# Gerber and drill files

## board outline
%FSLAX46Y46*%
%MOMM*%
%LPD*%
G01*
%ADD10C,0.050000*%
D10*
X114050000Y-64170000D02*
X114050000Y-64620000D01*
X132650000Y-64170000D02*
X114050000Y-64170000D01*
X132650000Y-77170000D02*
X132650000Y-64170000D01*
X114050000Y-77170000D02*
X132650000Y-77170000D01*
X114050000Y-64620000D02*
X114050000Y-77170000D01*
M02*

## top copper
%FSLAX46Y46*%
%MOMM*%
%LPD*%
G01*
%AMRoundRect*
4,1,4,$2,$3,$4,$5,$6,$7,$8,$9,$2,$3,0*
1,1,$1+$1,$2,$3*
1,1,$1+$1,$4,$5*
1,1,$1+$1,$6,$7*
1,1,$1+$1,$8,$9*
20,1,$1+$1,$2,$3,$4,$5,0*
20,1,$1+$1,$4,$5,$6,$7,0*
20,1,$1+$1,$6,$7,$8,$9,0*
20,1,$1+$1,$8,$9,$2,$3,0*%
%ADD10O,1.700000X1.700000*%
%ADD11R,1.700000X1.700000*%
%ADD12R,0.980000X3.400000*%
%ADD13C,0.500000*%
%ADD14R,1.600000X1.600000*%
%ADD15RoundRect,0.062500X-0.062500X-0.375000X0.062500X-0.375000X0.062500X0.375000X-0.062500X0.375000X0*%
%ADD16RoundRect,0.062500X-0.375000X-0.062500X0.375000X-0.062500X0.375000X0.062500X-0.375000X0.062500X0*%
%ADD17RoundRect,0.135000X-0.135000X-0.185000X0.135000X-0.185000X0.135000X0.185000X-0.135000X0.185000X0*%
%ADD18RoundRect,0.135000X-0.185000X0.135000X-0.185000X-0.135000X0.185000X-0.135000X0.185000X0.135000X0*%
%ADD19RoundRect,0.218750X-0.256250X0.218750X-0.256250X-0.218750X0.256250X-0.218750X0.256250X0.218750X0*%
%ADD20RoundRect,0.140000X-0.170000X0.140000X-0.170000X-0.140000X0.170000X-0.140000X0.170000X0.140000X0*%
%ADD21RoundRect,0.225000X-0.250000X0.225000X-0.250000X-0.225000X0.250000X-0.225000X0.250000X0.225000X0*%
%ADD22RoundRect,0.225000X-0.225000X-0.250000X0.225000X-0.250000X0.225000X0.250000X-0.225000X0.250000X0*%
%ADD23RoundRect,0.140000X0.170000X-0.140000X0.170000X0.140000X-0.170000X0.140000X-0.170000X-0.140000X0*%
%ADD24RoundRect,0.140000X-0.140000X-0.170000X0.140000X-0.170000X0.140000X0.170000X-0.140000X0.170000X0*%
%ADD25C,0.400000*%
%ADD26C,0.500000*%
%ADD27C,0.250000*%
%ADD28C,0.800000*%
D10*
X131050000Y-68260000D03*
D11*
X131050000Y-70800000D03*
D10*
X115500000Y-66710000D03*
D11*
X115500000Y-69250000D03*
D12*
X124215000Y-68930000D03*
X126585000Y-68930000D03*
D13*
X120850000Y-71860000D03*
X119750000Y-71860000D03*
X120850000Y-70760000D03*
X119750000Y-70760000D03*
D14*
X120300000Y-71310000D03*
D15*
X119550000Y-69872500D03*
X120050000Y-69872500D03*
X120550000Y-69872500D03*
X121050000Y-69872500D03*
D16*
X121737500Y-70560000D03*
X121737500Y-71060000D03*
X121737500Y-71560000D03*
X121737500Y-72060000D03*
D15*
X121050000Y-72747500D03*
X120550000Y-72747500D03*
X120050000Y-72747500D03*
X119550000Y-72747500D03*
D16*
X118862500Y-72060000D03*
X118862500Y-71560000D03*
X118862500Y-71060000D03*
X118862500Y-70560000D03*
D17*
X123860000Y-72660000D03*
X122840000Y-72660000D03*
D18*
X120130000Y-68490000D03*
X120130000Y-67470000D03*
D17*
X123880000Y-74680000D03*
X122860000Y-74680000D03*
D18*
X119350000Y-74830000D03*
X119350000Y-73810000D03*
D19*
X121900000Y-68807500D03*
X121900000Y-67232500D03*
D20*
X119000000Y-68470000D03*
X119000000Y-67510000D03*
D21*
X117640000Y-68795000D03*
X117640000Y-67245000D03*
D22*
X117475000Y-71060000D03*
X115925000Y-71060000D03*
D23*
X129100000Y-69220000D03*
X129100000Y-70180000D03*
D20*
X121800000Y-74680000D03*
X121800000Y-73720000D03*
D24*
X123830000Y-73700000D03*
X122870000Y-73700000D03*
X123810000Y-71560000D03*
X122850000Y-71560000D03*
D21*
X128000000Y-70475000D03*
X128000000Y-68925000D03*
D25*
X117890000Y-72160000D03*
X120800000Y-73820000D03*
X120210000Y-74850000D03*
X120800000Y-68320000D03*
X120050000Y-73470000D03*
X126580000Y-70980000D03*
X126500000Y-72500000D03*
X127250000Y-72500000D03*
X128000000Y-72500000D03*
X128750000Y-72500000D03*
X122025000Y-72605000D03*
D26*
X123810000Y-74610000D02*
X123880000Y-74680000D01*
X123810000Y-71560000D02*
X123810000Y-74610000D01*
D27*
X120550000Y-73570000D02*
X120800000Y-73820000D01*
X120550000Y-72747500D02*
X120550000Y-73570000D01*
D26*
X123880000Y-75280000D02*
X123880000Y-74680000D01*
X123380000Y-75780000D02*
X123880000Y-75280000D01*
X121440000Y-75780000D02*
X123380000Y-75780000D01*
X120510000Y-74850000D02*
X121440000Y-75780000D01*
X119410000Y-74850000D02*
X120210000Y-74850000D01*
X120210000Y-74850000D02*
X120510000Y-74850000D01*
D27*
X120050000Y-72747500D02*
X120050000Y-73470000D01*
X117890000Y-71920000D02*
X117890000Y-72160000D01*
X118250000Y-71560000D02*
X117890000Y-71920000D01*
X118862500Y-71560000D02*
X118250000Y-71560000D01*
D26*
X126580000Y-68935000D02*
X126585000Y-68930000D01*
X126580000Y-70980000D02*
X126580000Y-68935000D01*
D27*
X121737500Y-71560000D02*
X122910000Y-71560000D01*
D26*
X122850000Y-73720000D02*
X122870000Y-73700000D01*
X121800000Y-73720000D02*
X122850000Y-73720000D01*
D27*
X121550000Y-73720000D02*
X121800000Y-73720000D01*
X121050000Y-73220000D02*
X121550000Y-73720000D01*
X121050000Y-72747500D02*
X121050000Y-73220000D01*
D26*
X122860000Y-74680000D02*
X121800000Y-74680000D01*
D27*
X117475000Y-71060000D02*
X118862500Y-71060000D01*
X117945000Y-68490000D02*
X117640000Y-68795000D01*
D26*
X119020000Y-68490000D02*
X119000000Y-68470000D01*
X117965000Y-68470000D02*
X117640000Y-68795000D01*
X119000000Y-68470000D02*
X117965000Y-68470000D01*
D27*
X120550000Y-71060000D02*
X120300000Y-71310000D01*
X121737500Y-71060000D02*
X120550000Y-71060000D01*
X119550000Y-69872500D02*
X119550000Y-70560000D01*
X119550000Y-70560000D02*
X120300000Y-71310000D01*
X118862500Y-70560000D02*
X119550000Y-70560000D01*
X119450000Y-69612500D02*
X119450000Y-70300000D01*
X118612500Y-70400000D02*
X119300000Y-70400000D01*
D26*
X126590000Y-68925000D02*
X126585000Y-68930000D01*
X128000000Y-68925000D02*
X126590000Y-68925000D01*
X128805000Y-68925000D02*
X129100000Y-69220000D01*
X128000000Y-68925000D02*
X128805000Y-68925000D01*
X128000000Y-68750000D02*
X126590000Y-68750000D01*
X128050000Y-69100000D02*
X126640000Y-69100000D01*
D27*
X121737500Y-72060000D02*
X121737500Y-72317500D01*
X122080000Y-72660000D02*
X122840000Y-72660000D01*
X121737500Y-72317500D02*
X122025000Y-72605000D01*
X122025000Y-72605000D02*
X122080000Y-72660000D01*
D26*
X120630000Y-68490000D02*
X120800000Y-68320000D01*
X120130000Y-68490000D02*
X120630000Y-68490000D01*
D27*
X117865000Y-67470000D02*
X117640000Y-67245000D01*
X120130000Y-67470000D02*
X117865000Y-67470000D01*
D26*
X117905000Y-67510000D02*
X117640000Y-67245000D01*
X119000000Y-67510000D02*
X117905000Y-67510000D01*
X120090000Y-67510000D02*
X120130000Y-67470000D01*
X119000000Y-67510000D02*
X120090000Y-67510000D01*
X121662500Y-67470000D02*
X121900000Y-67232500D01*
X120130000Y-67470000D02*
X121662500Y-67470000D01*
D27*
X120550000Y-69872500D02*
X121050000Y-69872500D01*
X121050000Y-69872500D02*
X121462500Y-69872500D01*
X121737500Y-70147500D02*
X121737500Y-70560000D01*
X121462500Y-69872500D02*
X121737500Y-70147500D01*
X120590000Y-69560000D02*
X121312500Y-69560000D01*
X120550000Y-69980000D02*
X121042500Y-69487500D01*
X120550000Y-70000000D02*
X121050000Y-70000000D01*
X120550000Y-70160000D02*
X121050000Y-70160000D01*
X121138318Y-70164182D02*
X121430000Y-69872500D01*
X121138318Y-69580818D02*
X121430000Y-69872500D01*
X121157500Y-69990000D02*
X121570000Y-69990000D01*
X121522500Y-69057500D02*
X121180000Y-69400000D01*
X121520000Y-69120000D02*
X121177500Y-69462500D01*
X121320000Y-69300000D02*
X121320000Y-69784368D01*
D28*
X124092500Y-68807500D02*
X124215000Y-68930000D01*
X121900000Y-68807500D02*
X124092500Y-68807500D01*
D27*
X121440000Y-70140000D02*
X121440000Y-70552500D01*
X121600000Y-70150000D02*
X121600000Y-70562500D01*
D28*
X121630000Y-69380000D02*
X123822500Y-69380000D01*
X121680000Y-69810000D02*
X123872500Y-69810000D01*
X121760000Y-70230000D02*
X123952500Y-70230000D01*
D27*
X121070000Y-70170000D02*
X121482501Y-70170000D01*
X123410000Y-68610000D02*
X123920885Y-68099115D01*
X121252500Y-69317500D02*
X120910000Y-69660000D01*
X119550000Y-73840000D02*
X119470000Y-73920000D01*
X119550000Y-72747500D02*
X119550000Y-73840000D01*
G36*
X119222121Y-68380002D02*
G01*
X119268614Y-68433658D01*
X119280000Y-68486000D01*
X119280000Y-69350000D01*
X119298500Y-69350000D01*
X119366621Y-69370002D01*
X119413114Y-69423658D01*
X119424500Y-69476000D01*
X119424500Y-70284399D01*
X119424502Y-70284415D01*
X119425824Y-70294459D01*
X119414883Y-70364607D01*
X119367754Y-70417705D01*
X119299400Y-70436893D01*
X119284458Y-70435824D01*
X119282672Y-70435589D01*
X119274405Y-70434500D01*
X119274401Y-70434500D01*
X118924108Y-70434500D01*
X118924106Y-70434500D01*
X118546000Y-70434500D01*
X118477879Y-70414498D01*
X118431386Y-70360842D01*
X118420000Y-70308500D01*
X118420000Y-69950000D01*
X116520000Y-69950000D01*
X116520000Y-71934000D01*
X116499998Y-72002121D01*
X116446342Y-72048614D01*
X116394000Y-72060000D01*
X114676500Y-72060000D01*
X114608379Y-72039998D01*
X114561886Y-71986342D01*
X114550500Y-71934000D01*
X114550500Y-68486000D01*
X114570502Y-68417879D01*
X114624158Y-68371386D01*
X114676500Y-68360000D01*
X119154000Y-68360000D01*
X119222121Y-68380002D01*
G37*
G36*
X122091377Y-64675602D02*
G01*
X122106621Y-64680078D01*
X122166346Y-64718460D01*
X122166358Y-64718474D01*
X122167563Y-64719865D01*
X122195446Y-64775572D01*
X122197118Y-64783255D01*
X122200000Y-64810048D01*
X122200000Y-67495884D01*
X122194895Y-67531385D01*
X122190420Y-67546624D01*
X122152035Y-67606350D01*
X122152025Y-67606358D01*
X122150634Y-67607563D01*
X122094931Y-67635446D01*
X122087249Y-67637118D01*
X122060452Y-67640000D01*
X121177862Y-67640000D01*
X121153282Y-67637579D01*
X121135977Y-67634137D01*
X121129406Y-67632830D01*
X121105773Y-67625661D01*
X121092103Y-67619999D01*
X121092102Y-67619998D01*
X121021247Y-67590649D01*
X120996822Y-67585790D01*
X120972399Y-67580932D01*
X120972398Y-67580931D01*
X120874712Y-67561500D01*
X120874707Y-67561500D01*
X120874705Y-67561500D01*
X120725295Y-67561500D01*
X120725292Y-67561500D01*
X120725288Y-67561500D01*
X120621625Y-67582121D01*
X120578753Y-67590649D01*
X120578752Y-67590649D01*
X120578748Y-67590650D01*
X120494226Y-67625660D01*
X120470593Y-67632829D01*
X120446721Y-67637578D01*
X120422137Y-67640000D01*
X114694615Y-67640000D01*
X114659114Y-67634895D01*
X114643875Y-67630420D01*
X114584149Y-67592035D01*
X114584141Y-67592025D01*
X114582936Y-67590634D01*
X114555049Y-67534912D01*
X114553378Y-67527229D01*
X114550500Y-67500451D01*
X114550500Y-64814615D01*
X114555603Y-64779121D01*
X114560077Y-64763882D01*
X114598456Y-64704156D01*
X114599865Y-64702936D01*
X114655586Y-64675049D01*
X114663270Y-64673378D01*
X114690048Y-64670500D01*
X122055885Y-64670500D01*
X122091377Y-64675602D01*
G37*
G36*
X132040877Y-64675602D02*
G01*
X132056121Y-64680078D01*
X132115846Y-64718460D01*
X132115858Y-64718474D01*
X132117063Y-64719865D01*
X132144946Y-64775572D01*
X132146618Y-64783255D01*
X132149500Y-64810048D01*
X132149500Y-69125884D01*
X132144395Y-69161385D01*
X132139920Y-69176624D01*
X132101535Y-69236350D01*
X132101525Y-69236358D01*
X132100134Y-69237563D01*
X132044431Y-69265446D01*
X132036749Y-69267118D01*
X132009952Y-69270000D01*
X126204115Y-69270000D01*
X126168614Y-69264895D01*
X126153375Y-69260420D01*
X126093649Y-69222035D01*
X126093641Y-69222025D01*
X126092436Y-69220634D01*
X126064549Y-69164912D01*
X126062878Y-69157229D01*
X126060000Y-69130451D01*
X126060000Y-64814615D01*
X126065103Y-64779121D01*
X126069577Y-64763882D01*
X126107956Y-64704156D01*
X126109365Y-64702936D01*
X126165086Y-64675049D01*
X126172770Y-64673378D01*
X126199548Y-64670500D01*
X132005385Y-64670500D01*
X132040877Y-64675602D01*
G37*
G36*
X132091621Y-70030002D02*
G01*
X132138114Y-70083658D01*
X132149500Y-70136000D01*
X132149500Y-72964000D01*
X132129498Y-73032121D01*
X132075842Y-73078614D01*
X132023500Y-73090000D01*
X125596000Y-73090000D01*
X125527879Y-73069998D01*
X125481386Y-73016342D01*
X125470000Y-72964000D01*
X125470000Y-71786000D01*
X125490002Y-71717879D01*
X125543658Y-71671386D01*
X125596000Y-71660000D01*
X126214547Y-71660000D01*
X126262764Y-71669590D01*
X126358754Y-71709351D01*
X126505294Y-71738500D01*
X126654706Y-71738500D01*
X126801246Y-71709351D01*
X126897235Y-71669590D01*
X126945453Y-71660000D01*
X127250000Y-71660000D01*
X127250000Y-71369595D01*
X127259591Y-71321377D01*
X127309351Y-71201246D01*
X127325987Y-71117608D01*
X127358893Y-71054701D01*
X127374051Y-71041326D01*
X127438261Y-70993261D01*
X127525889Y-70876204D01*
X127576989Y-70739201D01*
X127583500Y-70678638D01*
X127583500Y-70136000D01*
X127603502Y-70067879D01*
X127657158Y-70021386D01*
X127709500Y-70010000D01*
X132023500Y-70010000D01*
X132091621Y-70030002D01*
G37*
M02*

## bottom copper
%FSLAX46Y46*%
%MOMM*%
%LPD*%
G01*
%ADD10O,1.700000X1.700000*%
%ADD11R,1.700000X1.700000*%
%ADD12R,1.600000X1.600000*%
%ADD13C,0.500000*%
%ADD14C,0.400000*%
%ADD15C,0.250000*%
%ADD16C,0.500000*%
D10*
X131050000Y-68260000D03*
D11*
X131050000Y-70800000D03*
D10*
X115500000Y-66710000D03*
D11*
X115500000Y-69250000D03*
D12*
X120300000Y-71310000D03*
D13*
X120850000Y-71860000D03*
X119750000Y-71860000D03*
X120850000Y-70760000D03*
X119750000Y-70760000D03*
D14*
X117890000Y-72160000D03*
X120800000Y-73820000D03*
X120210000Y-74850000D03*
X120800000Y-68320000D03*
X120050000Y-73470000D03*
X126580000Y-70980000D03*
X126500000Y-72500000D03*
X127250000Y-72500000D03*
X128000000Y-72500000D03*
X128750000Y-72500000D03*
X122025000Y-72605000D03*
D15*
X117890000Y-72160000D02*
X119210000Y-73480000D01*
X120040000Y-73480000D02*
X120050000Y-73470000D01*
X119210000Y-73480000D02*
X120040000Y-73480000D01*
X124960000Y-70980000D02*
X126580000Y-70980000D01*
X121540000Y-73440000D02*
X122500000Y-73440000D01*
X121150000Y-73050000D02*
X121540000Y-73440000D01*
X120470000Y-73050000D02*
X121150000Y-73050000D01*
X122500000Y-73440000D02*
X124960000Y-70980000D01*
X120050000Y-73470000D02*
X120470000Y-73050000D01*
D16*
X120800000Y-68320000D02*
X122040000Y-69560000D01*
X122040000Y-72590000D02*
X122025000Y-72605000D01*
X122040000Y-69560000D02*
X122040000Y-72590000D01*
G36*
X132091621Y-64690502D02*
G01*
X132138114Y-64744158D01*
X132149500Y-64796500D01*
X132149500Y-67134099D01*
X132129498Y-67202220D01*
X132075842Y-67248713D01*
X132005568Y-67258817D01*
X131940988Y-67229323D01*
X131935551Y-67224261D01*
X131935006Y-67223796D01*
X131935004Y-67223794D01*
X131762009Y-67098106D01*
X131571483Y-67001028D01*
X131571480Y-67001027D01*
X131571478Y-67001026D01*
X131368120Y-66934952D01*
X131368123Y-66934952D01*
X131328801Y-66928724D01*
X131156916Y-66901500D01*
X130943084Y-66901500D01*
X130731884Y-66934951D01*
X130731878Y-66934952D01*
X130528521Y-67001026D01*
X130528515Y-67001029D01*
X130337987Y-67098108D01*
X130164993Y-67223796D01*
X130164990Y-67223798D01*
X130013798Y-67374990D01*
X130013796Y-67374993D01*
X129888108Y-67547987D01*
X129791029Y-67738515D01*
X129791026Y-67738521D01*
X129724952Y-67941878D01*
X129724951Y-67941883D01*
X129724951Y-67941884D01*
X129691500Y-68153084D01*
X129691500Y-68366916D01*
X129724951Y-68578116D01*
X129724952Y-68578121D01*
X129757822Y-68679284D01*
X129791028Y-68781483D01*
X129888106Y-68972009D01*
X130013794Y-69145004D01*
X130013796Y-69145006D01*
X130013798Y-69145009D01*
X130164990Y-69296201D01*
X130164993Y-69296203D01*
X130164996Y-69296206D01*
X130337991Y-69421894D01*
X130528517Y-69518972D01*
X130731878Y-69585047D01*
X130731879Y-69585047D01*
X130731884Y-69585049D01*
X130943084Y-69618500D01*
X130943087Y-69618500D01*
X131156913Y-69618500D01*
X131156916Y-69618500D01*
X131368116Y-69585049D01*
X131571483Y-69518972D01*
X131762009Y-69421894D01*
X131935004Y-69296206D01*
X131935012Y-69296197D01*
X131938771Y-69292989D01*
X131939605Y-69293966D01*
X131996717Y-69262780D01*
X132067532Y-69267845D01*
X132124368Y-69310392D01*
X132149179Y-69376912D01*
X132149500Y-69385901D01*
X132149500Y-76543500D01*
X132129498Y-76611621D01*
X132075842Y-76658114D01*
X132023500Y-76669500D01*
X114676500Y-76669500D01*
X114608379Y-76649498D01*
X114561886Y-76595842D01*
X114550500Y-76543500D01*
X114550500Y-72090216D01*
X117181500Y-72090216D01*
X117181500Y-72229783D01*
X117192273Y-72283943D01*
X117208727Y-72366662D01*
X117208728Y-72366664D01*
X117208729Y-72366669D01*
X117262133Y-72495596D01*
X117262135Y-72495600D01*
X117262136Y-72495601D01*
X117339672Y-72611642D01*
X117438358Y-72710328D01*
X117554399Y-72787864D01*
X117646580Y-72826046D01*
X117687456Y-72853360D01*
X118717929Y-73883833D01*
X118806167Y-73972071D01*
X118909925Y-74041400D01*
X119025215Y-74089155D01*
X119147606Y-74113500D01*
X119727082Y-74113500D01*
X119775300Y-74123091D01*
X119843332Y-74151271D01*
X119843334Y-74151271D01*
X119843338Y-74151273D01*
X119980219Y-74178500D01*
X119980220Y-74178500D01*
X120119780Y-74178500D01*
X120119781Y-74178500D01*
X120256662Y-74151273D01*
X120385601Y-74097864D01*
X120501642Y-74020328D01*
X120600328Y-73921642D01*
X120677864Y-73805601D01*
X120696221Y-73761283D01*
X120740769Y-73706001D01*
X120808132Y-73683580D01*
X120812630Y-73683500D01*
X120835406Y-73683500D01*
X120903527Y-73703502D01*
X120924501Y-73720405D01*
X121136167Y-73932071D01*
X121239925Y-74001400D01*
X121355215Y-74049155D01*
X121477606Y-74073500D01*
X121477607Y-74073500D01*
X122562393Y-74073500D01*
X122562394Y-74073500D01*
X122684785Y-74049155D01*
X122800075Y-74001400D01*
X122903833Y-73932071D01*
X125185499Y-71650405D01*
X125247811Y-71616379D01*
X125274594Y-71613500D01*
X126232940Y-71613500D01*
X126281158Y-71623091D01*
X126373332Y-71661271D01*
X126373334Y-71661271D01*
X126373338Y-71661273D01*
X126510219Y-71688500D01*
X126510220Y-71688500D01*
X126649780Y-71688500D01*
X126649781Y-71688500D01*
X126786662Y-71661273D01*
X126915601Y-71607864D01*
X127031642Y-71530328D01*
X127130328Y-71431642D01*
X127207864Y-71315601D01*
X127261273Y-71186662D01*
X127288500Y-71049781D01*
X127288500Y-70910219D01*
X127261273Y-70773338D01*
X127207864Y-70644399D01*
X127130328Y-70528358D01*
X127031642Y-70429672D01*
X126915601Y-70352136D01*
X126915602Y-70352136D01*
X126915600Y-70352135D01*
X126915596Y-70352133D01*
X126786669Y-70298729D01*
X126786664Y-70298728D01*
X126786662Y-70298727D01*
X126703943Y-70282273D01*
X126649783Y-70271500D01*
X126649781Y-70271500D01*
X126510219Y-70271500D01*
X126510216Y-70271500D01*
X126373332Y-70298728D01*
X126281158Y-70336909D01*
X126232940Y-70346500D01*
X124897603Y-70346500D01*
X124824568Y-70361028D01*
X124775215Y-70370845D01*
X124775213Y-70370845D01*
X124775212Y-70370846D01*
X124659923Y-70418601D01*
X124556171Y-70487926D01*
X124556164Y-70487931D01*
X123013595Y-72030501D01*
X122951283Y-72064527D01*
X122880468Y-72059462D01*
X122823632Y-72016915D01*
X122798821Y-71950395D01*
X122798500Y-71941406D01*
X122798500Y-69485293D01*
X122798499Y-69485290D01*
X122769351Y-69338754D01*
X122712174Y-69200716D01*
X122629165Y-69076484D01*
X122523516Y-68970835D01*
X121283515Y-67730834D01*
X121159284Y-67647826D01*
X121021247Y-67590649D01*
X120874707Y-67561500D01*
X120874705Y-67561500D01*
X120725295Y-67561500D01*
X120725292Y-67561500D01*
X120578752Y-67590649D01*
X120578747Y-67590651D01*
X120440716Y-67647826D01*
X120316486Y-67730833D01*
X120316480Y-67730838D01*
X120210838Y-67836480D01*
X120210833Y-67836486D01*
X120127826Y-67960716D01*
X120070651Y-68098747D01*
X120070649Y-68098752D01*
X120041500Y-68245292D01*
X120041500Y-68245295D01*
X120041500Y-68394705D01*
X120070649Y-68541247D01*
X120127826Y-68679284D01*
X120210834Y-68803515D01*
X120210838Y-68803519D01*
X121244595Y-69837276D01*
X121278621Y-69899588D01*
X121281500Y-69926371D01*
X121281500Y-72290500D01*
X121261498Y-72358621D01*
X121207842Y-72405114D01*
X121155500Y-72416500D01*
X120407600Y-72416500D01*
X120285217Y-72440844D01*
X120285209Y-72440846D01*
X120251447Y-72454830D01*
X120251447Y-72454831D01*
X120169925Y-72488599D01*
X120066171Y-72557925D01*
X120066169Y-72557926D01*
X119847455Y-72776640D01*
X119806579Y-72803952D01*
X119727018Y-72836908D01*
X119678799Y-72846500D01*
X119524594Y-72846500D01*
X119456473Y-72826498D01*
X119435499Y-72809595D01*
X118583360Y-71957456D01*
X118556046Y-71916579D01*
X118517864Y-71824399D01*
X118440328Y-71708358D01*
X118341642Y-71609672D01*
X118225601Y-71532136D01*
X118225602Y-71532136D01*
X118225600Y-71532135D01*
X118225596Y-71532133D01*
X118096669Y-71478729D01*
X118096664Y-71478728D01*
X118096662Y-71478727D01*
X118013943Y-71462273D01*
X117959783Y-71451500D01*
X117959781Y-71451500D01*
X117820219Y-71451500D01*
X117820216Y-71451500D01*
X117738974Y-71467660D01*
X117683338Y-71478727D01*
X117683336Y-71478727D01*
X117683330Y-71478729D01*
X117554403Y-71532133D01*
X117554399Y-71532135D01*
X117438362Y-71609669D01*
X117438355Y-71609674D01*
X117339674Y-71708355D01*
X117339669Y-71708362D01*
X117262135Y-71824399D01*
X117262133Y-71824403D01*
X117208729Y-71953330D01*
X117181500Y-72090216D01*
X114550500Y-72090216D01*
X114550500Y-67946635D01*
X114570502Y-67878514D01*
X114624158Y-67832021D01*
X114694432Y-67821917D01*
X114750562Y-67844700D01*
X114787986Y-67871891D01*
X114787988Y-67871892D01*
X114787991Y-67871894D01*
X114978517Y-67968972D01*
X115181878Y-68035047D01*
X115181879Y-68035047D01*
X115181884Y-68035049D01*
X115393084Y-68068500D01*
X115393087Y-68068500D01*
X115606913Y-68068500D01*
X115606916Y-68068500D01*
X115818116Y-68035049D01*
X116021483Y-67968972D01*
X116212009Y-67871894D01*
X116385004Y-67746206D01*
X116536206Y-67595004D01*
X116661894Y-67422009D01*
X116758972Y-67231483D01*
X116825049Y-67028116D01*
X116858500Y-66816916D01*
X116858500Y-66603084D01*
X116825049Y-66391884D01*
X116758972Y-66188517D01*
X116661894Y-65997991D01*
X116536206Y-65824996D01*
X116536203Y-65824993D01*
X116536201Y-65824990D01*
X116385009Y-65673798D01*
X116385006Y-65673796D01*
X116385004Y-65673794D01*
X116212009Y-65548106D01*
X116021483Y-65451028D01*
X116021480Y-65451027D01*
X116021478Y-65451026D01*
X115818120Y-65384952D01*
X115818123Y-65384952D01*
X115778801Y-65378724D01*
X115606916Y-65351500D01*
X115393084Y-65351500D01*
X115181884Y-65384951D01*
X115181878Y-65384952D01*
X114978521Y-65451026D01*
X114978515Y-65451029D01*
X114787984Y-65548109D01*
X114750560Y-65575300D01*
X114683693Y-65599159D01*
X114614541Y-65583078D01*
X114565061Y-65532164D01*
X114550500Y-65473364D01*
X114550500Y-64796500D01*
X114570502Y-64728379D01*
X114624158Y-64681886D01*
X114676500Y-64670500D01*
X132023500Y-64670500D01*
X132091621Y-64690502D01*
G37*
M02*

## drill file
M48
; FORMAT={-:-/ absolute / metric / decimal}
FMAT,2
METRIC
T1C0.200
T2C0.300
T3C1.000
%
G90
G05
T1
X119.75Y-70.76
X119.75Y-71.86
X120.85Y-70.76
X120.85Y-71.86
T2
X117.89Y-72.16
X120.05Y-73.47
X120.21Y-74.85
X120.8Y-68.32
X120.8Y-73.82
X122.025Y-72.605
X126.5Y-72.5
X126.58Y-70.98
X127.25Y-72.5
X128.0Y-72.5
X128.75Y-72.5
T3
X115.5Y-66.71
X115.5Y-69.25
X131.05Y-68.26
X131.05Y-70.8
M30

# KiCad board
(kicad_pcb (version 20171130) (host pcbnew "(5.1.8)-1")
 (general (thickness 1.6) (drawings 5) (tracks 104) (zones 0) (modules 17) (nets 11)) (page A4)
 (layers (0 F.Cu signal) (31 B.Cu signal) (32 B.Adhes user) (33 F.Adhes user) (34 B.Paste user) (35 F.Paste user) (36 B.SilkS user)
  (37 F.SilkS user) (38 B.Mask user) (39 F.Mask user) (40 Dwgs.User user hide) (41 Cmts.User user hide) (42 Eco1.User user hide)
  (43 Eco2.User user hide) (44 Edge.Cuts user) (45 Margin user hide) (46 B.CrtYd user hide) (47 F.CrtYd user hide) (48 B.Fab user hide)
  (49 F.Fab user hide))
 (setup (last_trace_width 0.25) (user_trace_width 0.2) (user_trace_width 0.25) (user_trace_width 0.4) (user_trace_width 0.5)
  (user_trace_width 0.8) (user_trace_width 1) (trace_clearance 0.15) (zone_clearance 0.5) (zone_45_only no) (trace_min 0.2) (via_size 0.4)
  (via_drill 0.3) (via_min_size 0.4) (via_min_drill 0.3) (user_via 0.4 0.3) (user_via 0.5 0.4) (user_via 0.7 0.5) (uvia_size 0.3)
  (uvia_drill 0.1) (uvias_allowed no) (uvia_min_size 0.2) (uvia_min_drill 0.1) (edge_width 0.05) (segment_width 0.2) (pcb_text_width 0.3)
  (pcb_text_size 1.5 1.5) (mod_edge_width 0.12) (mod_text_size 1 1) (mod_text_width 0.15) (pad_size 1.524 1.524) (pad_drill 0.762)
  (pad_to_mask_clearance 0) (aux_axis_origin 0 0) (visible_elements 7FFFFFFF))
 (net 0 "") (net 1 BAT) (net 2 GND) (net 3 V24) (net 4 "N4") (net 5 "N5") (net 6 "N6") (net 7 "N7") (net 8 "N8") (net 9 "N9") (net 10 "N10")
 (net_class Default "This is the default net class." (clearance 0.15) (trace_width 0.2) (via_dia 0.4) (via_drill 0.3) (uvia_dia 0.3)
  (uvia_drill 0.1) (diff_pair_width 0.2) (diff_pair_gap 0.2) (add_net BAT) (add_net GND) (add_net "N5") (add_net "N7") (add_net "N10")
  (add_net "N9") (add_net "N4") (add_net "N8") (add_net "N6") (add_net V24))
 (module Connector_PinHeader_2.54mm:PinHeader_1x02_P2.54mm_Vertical (layer F.Cu) (at 131.05 70.8 180)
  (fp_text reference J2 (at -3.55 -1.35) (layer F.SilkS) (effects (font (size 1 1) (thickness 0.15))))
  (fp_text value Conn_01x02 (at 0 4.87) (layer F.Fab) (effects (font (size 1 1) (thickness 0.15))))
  (pad 2 thru_hole oval (at 0 2.54 180) (size 1.7 1.7) (drill 1) (layers *.Cu *.Mask) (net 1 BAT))
  (pad 1 thru_hole rect (at 0 0 180) (size 1.7 1.7) (drill 1) (layers *.Cu *.Mask) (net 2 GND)))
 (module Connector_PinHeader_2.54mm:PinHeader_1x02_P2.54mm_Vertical (layer F.Cu) (at 115.5 69.25 180)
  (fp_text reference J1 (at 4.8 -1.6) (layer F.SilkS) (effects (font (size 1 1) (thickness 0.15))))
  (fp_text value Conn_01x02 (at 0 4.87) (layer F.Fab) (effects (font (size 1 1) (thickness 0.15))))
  (pad 2 thru_hole oval (at 0 2.54 180) (size 1.7 1.7) (drill 1) (layers *.Cu *.Mask) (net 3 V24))
  (pad 1 thru_hole rect (at 0 0 180) (size 1.7 1.7) (drill 1) (layers *.Cu *.Mask) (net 2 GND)))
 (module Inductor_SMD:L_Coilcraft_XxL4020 (layer F.Cu) (at 125.4 68.93 180)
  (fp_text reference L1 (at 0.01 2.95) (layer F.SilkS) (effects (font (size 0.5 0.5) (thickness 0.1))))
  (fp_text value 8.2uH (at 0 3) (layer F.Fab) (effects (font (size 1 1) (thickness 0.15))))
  (pad 2 smd rect (at 1.185 0 180) (size 0.98 3.4) (layers F.Cu F.Paste F.Mask) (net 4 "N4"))
  (pad 1 smd rect (at -1.185 0 180) (size 0.98 3.4) (layers F.Cu F.Paste F.Mask) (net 1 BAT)))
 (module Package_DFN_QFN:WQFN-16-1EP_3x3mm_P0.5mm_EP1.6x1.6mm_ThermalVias (layer F.Cu) (at 120.3 71.31)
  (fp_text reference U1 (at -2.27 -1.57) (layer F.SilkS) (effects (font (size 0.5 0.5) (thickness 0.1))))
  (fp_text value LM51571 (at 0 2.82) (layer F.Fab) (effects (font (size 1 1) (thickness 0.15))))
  (pad "" smd roundrect (at 0.4 0.4) (size 0.69 0.69) (layers F.Paste) (roundrect_rratio 0.25))
  (pad "" smd roundrect (at 0.4 -0.4) (size 0.69 0.69) (layers F.Paste) (roundrect_rratio 0.25))
  (pad "" smd roundrect (at -0.4 0.4) (size 0.69 0.69) (layers F.Paste) (roundrect_rratio 0.25))
  (pad "" smd roundrect (at -0.4 -0.4) (size 0.69 0.69) (layers F.Paste) (roundrect_rratio 0.25))
  (pad 17 smd rect (at 0 0) (size 1.6 1.6) (layers B.Cu) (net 2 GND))
  (pad 17 thru_hole circle (at 0.55 0.55) (size 0.5 0.5) (drill 0.2) (layers *.Cu) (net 2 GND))
  (pad 17 thru_hole circle (at -0.55 0.55) (size 0.5 0.5) (drill 0.2) (layers *.Cu) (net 2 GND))
  (pad 17 thru_hole circle (at 0.55 -0.55) (size 0.5 0.5) (drill 0.2) (layers *.Cu) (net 2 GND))
  (pad 17 thru_hole circle (at -0.55 -0.55) (size 0.5 0.5) (drill 0.2) (layers *.Cu) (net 2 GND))
  (pad 17 smd rect (at 0 0) (size 1.6 1.6) (layers F.Cu F.Mask) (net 2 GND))
  (pad 16 smd roundrect (at -0.75 -1.4375) (size 0.25 0.875) (layers F.Cu F.Paste F.Mask) (roundrect_rratio 0.25) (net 2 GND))
  (pad 15 smd roundrect (at -0.25 -1.4375) (size 0.25 0.875) (layers F.Cu F.Paste F.Mask) (roundrect_rratio 0.25))
  (pad 14 smd roundrect (at 0.25 -1.4375) (size 0.25 0.875) (layers F.Cu F.Paste F.Mask) (roundrect_rratio 0.25) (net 4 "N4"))
  (pad 13 smd roundrect (at 0.75 -1.4375) (size 0.25 0.875) (layers F.Cu F.Paste F.Mask) (roundrect_rratio 0.25) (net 4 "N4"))
  (pad 12 smd roundrect (at 1.4375 -0.75) (size 0.875 0.25) (layers F.Cu F.Paste F.Mask) (roundrect_rratio 0.25) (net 4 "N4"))
  (pad 11 smd roundrect (at 1.4375 -0.25) (size 0.875 0.25) (layers F.Cu F.Paste F.Mask) (roundrect_rratio 0.25) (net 2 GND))
  (pad 10 smd roundrect (at 1.4375 0.25) (size 0.875 0.25) (layers F.Cu F.Paste F.Mask) (roundrect_rratio 0.25) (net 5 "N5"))
  (pad 9 smd roundrect (at 1.4375 0.75) (size 0.875 0.25) (layers F.Cu F.Paste F.Mask) (roundrect_rratio 0.25) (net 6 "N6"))
  (pad 8 smd roundrect (at 0.75 1.4375) (size 0.25 0.875) (layers F.Cu F.Paste F.Mask) (roundrect_rratio 0.25) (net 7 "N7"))
  (pad 7 smd roundrect (at 0.25 1.4375) (size 0.25 0.875) (layers F.Cu F.Paste F.Mask) (roundrect_rratio 0.25) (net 2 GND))
  (pad 6 smd roundrect (at -0.25 1.4375) (size 0.25 0.875) (layers F.Cu F.Paste F.Mask) (roundrect_rratio 0.25) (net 1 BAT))
  (pad 5 smd roundrect (at -0.75 1.4375) (size 0.25 0.875) (layers F.Cu F.Paste F.Mask) (roundrect_rratio 0.25) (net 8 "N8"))
  (pad 4 smd roundrect (at -1.4375 0.75) (size 0.875 0.25) (layers F.Cu F.Paste F.Mask) (roundrect_rratio 0.25))
  (pad 3 smd roundrect (at -1.4375 0.25) (size 0.875 0.25) (layers F.Cu F.Paste F.Mask) (roundrect_rratio 0.25) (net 1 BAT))
  (pad 2 smd roundrect (at -1.4375 -0.25) (size 0.875 0.25) (layers F.Cu F.Paste F.Mask) (roundrect_rratio 0.25) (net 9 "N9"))
  (pad 1 smd roundrect (at -1.4375 -0.75) (size 0.875 0.25) (layers F.Cu F.Paste F.Mask) (roundrect_rratio 0.25) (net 2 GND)))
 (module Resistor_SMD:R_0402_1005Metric (layer F.Cu) (at 123.35 72.66)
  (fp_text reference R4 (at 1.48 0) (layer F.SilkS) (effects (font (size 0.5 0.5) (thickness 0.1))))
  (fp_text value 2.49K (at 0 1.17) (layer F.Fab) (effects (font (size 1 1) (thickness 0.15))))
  (pad 2 smd roundrect (at 0.51 0) (size 0.54 0.64) (layers F.Cu F.Paste F.Mask) (roundrect_rratio 0.25) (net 2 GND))
  (pad 1 smd roundrect (at -0.51 0) (size 0.54 0.64) (layers F.Cu F.Paste F.Mask) (roundrect_rratio 0.25) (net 6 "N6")))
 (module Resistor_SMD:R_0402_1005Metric (layer F.Cu) (at 120.13 67.98 270)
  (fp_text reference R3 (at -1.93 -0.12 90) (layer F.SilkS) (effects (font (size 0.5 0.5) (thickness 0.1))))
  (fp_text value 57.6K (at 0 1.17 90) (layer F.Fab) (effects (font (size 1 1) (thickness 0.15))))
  (pad 2 smd roundrect (at 0.51 0 270) (size 0.54 0.64) (layers F.Cu F.Paste F.Mask) (roundrect_rratio 0.25) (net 6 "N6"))
  (pad 1 smd roundrect (at -0.51 0 270) (size 0.54 0.64) (layers F.Cu F.Paste F.Mask) (roundrect_rratio 0.25) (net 3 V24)))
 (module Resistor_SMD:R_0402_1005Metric (layer F.Cu) (at 123.37 74.68)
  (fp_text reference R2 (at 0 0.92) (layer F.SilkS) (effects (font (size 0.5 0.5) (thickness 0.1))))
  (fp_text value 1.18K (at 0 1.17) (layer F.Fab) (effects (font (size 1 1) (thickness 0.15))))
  (pad 2 smd roundrect (at 0.51 0) (size 0.54 0.64) (layers F.Cu F.Paste F.Mask) (roundrect_rratio 0.25) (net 2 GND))
  (pad 1 smd roundrect (at -0.51 0) (size 0.54 0.64) (layers F.Cu F.Paste F.Mask) (roundrect_rratio 0.25) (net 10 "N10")))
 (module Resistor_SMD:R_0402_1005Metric (layer F.Cu) (at 119.35 74.32 270)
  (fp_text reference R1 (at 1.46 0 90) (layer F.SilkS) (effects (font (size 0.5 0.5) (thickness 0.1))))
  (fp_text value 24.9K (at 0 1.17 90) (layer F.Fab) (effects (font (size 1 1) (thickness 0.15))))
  (pad 2 smd roundrect (at 0.51 0 270) (size 0.54 0.64) (layers F.Cu F.Paste F.Mask) (roundrect_rratio 0.25) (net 2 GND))
  (pad 1 smd roundrect (at -0.51 0 270) (size 0.54 0.64) (layers F.Cu F.Paste F.Mask) (roundrect_rratio 0.25) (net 8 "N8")))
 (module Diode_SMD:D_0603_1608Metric (layer F.Cu) (at 121.9 68.02 270)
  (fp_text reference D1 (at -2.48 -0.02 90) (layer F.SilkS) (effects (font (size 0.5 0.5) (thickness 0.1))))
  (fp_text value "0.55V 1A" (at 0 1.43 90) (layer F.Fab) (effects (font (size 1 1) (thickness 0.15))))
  (pad 2 smd roundrect (at 0.7875 0 270) (size 0.875 0.95) (layers F.Cu F.Paste F.Mask) (roundrect_rratio 0.25) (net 4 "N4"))
  (pad 1 smd roundrect (at -0.7875 0 270) (size 0.875 0.95) (layers F.Cu F.Paste F.Mask) (roundrect_rratio 0.25) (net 3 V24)))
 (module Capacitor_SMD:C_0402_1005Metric (layer F.Cu) (at 119 67.99 270)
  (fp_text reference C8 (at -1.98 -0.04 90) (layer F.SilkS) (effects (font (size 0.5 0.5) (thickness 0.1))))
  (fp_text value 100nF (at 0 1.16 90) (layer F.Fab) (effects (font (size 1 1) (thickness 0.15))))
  (pad 2 smd roundrect (at 0.48 0 270) (size 0.56 0.62) (layers F.Cu F.Paste F.Mask) (roundrect_rratio 0.25) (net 2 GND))
  (pad 1 smd roundrect (at -0.48 0 270) (size 0.56 0.62) (layers F.Cu F.Paste F.Mask) (roundrect_rratio 0.25) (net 3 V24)))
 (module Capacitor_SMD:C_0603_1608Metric (layer F.Cu) (at 117.64 68.02 270)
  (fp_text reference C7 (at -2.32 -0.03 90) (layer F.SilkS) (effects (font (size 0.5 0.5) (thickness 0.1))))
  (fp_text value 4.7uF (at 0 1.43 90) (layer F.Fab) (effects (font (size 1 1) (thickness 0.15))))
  (pad 2 smd roundrect (at 0.775 0 270) (size 0.9 0.95) (layers F.Cu F.Paste F.Mask) (roundrect_rratio 0.25) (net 2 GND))
  (pad 1 smd roundrect (at -0.775 0 270) (size 0.9 0.95) (layers F.Cu F.Paste F.Mask) (roundrect_rratio 0.25) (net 3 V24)))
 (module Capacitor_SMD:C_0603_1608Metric (layer F.Cu) (at 116.7 71.06)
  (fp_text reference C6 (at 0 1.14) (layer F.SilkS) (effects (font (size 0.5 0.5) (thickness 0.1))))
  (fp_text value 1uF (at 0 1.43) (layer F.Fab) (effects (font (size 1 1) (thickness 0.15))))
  (pad 2 smd roundrect (at 0.775 0) (size 0.9 0.95) (layers F.Cu F.Paste F.Mask) (roundrect_rratio 0.25) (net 9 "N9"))
  (pad 1 smd roundrect (at -0.775 0) (size 0.9 0.95) (layers F.Cu F.Paste F.Mask) (roundrect_rratio 0.25) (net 2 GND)))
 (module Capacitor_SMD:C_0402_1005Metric (layer F.Cu) (at 129.1 69.7 90)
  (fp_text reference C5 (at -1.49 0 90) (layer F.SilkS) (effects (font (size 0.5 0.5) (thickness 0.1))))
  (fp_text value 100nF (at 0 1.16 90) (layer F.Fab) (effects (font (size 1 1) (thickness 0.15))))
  (pad 2 smd roundrect (at 0.48 0 90) (size 0.56 0.62) (layers F.Cu F.Paste F.Mask) (roundrect_rratio 0.25) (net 1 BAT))
  (pad 1 smd roundrect (at -0.48 0 90) (size 0.56 0.62) (layers F.Cu F.Paste F.Mask) (roundrect_rratio 0.25) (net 2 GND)))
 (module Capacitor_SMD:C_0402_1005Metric (layer F.Cu) (at 121.8 74.2 270)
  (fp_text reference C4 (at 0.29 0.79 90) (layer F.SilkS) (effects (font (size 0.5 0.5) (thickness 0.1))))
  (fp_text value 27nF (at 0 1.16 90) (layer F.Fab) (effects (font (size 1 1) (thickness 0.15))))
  (pad 2 smd roundrect (at 0.48 0 270) (size 0.56 0.62) (layers F.Cu F.Paste F.Mask) (roundrect_rratio 0.25) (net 10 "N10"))
  (pad 1 smd roundrect (at -0.48 0 270) (size 0.56 0.62) (layers F.Cu F.Paste F.Mask) (roundrect_rratio 0.25) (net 7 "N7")))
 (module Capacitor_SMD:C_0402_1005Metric (layer F.Cu) (at 123.35 73.7)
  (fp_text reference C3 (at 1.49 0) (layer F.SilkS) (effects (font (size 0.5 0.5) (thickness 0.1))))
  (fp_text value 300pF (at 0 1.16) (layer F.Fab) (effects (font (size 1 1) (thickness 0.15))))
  (pad 2 smd roundrect (at 0.48 0) (size 0.56 0.62) (layers F.Cu F.Paste F.Mask) (roundrect_rratio 0.25) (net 2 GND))
  (pad 1 smd roundrect (at -0.48 0) (size 0.56 0.62) (layers F.Cu F.Paste F.Mask) (roundrect_rratio 0.25) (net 7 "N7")))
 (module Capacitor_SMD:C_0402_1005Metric (layer F.Cu) (at 123.33 71.56)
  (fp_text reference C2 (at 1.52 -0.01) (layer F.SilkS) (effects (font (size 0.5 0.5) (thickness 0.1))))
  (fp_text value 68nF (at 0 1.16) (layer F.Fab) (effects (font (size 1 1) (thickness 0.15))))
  (pad 2 smd roundrect (at 0.48 0) (size 0.56 0.62) (layers F.Cu F.Paste F.Mask) (roundrect_rratio 0.25) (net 2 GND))
  (pad 1 smd roundrect (at -0.48 0) (size 0.56 0.62) (layers F.Cu F.Paste F.Mask) (roundrect_rratio 0.25) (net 5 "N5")))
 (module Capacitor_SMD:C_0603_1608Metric (layer F.Cu) (at 128 69.7 270)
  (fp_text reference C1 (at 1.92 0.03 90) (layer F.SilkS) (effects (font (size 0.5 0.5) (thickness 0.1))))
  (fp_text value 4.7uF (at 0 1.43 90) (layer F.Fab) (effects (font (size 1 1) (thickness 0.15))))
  (pad 2 smd roundrect (at 0.775 0 270) (size 0.9 0.95) (layers F.Cu F.Paste F.Mask) (roundrect_rratio 0.25) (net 2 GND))
  (pad 1 smd roundrect (at -0.775 0 270) (size 0.9 0.95) (layers F.Cu F.Paste F.Mask) (roundrect_rratio 0.25) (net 1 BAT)))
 (gr_line (start 114.05 64.17) (end 114.05 64.62) (layer Edge.Cuts) (width 0.05))
 (gr_line (start 132.65 64.17) (end 114.05 64.17) (layer Edge.Cuts) (width 0.05))
 (gr_line (start 132.65 77.17) (end 132.65 64.17) (layer Edge.Cuts) (width 0.05))
 (gr_line (start 114.05 77.17) (end 132.65 77.17) (layer Edge.Cuts) (width 0.05))
 (gr_line (start 114.05 64.62) (end 114.05 77.17) (layer Edge.Cuts) (width 0.05))
 (via (at 117.89 72.16) (size 0.4) (drill 0.3) (layers F.Cu B.Cu) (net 1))
 (segment (start 123.81 74.61) (end 123.88 74.68) (width 0.5) (layer F.Cu) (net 2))
 (segment (start 123.81 71.56) (end 123.81 74.61) (width 0.5) (layer F.Cu) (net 2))
 (segment (start 120.55 73.57) (end 120.8 73.82) (width 0.25) (layer F.Cu) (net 2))
 (segment (start 120.55 72.7475) (end 120.55 73.57) (width 0.25) (layer F.Cu) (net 2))
 (via (at 120.8 73.82) (size 0.4) (drill 0.3) (layers F.Cu B.Cu) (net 2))
 (segment (start 123.88 75.28) (end 123.88 74.68) (width 0.5) (layer F.Cu) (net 2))
 (segment (start 123.38 75.78) (end 123.88 75.28) (width 0.5) (layer F.Cu) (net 2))
 (segment (start 121.44 75.78) (end 123.38 75.78) (width 0.5) (layer F.Cu) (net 2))
 (segment (start 120.51 74.85) (end 121.44 75.78) (width 0.5) (layer F.Cu) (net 2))
 (segment (start 119.41 74.85) (end 120.21 74.85) (width 0.5) (layer F.Cu) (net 2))
 (segment (start 120.21 74.85) (end 120.51 74.85) (width 0.5) (layer F.Cu) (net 2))
 (via (at 120.21 74.85) (size 0.4) (drill 0.3) (layers F.Cu B.Cu) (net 2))
 (via (at 120.8 68.32) (size 0.4) (drill 0.3) (layers F.Cu B.Cu) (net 6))
 (via (at 120.05 73.47) (size 0.4) (drill 0.3) (layers F.Cu B.Cu) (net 1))
 (segment (start 120.05 72.7475) (end 120.05 73.47) (width 0.25) (layer F.Cu) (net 1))
 (via (at 126.58 70.98) (size 0.4) (drill 0.3) (layers F.Cu B.Cu) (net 1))
 (segment (start 117.89 71.92) (end 117.89 72.16) (width 0.25) (layer F.Cu) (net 1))
 (segment (start 118.25 71.56) (end 117.89 71.92) (width 0.25) (layer F.Cu) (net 1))
 (segment (start 118.8625 71.56) (end 118.25 71.56) (width 0.25) (layer F.Cu) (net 1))
 (segment (start 117.89 72.16) (end 119.21 73.48) (width 0.25) (layer B.Cu) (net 1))
 (segment (start 120.04 73.48) (end 120.05 73.47) (width 0.25) (layer B.Cu) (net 1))
 (segment (start 119.21 73.48) (end 120.04 73.48) (width 0.25) (layer B.Cu) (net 1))
 (segment (start 126.58 68.935) (end 126.585 68.93) (width 0.5) (layer F.Cu) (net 1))
 (segment (start 126.58 70.98) (end 126.58 68.935) (width 0.5) (layer F.Cu) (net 1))
 (segment (start 124.96 70.98) (end 126.58 70.98) (width 0.25) (layer B.Cu) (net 1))
 (segment (start 121.54 73.44) (end 122.5 73.44) (width 0.25) (layer B.Cu) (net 1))
 (segment (start 121.15 73.05) (end 121.54 73.44) (width 0.25) (layer B.Cu) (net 1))
 (segment (start 120.47 73.05) (end 121.15 73.05) (width 0.25) (layer B.Cu) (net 1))
 (segment (start 122.5 73.44) (end 124.96 70.98) (width 0.25) (layer B.Cu) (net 1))
 (segment (start 120.05 73.47) (end 120.47 73.05) (width 0.25) (layer B.Cu) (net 1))
 (segment (start 121.7375 71.56) (end 122.91 71.56) (width 0.25) (layer F.Cu) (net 5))
 (segment (start 122.85 73.72) (end 122.87 73.7) (width 0.5) (layer F.Cu) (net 7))
 (segment (start 121.8 73.72) (end 122.85 73.72) (width 0.5) (layer F.Cu) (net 7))
 (segment (start 121.55 73.72) (end 121.8 73.72) (width 0.25) (layer F.Cu) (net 7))
 (segment (start 121.05 73.22) (end 121.55 73.72) (width 0.25) (layer F.Cu) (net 7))
 (segment (start 121.05 72.7475) (end 121.05 73.22) (width 0.25) (layer F.Cu) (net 7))
 (segment (start 122.86 74.68) (end 121.8 74.68) (width 0.5) (layer F.Cu) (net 10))
 (segment (start 117.475 71.06) (end 118.8625 71.06) (width 0.25) (layer F.Cu) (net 9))
 (segment (start 117.945 68.49) (end 117.64 68.795) (width 0.25) (layer F.Cu) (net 2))
 (segment (start 119.02 68.49) (end 119 68.47) (width 0.5) (layer F.Cu) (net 2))
 (segment (start 117.965 68.47) (end 117.64 68.795) (width 0.5) (layer F.Cu) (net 2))
 (segment (start 119 68.47) (end 117.965 68.47) (width 0.5) (layer F.Cu) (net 2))
 (segment (start 120.55 71.06) (end 120.3 71.31) (width 0.25) (layer F.Cu) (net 2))
 (segment (start 121.7375 71.06) (end 120.55 71.06) (width 0.25) (layer F.Cu) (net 2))
 (via (at 126.5 72.5) (size 0.4) (drill 0.3) (layers F.Cu B.Cu) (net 2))
 (via (at 127.25 72.5) (size 0.4) (drill 0.3) (layers F.Cu B.Cu) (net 2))
 (via (at 128 72.5) (size 0.4) (drill 0.3) (layers F.Cu B.Cu) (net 2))
 (via (at 128.75 72.5) (size 0.4) (drill 0.3) (layers F.Cu B.Cu) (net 2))
 (segment (start 119.55 69.8725) (end 119.55 70.56) (width 0.25) (layer F.Cu) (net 2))
 (segment (start 119.55 70.56) (end 120.3 71.31) (width 0.25) (layer F.Cu) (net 2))
 (segment (start 118.8625 70.56) (end 119.55 70.56) (width 0.25) (layer F.Cu) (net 2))
 (segment (start 119.45 69.6125) (end 119.45 70.3) (width 0.25) (layer F.Cu) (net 2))
 (segment (start 118.6125 70.4) (end 119.3 70.4) (width 0.25) (layer F.Cu) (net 2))
 (segment (start 126.59 68.925) (end 126.585 68.93) (width 0.5) (layer F.Cu) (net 1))
 (segment (start 128 68.925) (end 126.59 68.925) (width 0.5) (layer F.Cu) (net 1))
 (segment (start 128.805 68.925) (end 129.1 69.22) (width 0.5) (layer F.Cu) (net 1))
 (segment (start 128 68.925) (end 128.805 68.925) (width 0.5) (layer F.Cu) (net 1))
 (segment (start 128 68.75) (end 126.59 68.75) (width 0.5) (layer F.Cu) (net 1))
 (segment (start 128.05 69.1) (end 126.64 69.1) (width 0.5) (layer F.Cu) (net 1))
 (segment (start 121.7375 72.06) (end 121.7375 72.3175) (width 0.25) (layer F.Cu) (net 6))
 (segment (start 122.08 72.66) (end 122.84 72.66) (width 0.25) (layer F.Cu) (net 6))
 (segment (start 121.7375 72.3175) (end 122.025 72.605) (width 0.25) (layer F.Cu) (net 6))
 (segment (start 122.025 72.605) (end 122.08 72.66) (width 0.25) (layer F.Cu) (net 6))
 (via (at 122.025 72.605) (size 0.4) (drill 0.3) (layers F.Cu B.Cu) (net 6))
 (segment (start 120.63 68.49) (end 120.8 68.32) (width 0.5) (layer F.Cu) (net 6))
 (segment (start 120.13 68.49) (end 120.63 68.49) (width 0.5) (layer F.Cu) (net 6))
 (segment (start 120.8 68.32) (end 122.04 69.56) (width 0.5) (layer B.Cu) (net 6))
 (segment (start 122.04 72.59) (end 122.025 72.605) (width 0.5) (layer B.Cu) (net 6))
 (segment (start 122.04 69.56) (end 122.04 72.59) (width 0.5) (layer B.Cu) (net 6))
 (segment (start 117.865 67.47) (end 117.64 67.245) (width 0.25) (layer F.Cu) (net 3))
 (segment (start 120.13 67.47) (end 117.865 67.47) (width 0.25) (layer F.Cu) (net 3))
 (segment (start 117.905 67.51) (end 117.64 67.245) (width 0.5) (layer F.Cu) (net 3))
 (segment (start 119 67.51) (end 117.905 67.51) (width 0.5) (layer F.Cu) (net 3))
 (segment (start 120.09 67.51) (end 120.13 67.47) (width 0.5) (layer F.Cu) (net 3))
 (segment (start 119 67.51) (end 120.09 67.51) (width 0.5) (layer F.Cu) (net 3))
 (segment (start 121.6625 67.47) (end 121.9 67.2325) (width 0.5) (layer F.Cu) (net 3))
 (segment (start 120.13 67.47) (end 121.6625 67.47) (width 0.5) (layer F.Cu) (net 3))
 (segment (start 120.55 69.8725) (end 121.05 69.8725) (width 0.25) (layer F.Cu) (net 4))
 (segment (start 121.05 69.8725) (end 121.4625 69.8725) (width 0.25) (layer F.Cu) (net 4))
 (segment (start 121.7375 70.1475) (end 121.7375 70.56) (width 0.25) (layer F.Cu) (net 4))
 (segment (start 121.4625 69.8725) (end 121.7375 70.1475) (width 0.25) (layer F.Cu) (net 4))
 (segment (start 120.59 69.56) (end 121.3125 69.56) (width 0.25) (layer F.Cu) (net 4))
 (segment (start 120.55 69.98) (end 121.0425 69.4875) (width 0.25) (layer F.Cu) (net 4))
 (segment (start 120.55 70) (end 121.05 70) (width 0.25) (layer F.Cu) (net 4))
 (segment (start 120.55 70.16) (end 121.05 70.16) (width 0.25) (layer F.Cu) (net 4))
 (segment (start 121.138318 70.164182) (end 121.43 69.8725) (width 0.25) (layer F.Cu) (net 4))
 (segment (start 121.138318 69.580818) (end 121.43 69.8725) (width 0.25) (layer F.Cu) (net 4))
 (segment (start 121.1575 69.99) (end 121.57 69.99) (width 0.25) (layer F.Cu) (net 4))
 (segment (start 121.5225 69.0575) (end 121.18 69.4) (width 0.25) (layer F.Cu) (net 4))
 (segment (start 121.52 69.12) (end 121.1775 69.4625) (width 0.25) (layer F.Cu) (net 4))
 (segment (start 121.32 69.3) (end 121.32 69.784368) (width 0.25) (layer F.Cu) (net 4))
 (segment (start 124.0925 68.8075) (end 124.215 68.93) (width 0.8) (layer F.Cu) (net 4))
 (segment (start 121.9 68.8075) (end 124.0925 68.8075) (width 0.8) (layer F.Cu) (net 4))
 (segment (start 121.44 70.14) (end 121.44 70.5525) (width 0.25) (layer F.Cu) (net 4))
 (segment (start 121.6 70.15) (end 121.6 70.5625) (width 0.25) (layer F.Cu) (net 4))
 (segment (start 121.63 69.38) (end 123.8225 69.38) (width 0.8) (layer F.Cu) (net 4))
 (segment (start 121.68 69.81) (end 123.8725 69.81) (width 0.8) (layer F.Cu) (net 4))
 (segment (start 121.76 70.23) (end 123.9525 70.23) (width 0.8) (layer F.Cu) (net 4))
 (segment (start 121.07 70.17) (end 121.482501 70.17) (width 0.25) (layer F.Cu) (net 4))
 (segment (start 123.41 68.61) (end 123.920885 68.099115) (width 0.25) (layer F.Cu) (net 4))
 (segment (start 121.2525 69.3175) (end 120.91 69.66) (width 0.25) (layer F.Cu) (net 4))
 (segment (start 119.55 73.84) (end 119.47 73.92) (width 0.25) (layer F.Cu) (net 8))
 (segment (start 119.55 72.7475) (end 119.55 73.84) (width 0.25) (layer F.Cu) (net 8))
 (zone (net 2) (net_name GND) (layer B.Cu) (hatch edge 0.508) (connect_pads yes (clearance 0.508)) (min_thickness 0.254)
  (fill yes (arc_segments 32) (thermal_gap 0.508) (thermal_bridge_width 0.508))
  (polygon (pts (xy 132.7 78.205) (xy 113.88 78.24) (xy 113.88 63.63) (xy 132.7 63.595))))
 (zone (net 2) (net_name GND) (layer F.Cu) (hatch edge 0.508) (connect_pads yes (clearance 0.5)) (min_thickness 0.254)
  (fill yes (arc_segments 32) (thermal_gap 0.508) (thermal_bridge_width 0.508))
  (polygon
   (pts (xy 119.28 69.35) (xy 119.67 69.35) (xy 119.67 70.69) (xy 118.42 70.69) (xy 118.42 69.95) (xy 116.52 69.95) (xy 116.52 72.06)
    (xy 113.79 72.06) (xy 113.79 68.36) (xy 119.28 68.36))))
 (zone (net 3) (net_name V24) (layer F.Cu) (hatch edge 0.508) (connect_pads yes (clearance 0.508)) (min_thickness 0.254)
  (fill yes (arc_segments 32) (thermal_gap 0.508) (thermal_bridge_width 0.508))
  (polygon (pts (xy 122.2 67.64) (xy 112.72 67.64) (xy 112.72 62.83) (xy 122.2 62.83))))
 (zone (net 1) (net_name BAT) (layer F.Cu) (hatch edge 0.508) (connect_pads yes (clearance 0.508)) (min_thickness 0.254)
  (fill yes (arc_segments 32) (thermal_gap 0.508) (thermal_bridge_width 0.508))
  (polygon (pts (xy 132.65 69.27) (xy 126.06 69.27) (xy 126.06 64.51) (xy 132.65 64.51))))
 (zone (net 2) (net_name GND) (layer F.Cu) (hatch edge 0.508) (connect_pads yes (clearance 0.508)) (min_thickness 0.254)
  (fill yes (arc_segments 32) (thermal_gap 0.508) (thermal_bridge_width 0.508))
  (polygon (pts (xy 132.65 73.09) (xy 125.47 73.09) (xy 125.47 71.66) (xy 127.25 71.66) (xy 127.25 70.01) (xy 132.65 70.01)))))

